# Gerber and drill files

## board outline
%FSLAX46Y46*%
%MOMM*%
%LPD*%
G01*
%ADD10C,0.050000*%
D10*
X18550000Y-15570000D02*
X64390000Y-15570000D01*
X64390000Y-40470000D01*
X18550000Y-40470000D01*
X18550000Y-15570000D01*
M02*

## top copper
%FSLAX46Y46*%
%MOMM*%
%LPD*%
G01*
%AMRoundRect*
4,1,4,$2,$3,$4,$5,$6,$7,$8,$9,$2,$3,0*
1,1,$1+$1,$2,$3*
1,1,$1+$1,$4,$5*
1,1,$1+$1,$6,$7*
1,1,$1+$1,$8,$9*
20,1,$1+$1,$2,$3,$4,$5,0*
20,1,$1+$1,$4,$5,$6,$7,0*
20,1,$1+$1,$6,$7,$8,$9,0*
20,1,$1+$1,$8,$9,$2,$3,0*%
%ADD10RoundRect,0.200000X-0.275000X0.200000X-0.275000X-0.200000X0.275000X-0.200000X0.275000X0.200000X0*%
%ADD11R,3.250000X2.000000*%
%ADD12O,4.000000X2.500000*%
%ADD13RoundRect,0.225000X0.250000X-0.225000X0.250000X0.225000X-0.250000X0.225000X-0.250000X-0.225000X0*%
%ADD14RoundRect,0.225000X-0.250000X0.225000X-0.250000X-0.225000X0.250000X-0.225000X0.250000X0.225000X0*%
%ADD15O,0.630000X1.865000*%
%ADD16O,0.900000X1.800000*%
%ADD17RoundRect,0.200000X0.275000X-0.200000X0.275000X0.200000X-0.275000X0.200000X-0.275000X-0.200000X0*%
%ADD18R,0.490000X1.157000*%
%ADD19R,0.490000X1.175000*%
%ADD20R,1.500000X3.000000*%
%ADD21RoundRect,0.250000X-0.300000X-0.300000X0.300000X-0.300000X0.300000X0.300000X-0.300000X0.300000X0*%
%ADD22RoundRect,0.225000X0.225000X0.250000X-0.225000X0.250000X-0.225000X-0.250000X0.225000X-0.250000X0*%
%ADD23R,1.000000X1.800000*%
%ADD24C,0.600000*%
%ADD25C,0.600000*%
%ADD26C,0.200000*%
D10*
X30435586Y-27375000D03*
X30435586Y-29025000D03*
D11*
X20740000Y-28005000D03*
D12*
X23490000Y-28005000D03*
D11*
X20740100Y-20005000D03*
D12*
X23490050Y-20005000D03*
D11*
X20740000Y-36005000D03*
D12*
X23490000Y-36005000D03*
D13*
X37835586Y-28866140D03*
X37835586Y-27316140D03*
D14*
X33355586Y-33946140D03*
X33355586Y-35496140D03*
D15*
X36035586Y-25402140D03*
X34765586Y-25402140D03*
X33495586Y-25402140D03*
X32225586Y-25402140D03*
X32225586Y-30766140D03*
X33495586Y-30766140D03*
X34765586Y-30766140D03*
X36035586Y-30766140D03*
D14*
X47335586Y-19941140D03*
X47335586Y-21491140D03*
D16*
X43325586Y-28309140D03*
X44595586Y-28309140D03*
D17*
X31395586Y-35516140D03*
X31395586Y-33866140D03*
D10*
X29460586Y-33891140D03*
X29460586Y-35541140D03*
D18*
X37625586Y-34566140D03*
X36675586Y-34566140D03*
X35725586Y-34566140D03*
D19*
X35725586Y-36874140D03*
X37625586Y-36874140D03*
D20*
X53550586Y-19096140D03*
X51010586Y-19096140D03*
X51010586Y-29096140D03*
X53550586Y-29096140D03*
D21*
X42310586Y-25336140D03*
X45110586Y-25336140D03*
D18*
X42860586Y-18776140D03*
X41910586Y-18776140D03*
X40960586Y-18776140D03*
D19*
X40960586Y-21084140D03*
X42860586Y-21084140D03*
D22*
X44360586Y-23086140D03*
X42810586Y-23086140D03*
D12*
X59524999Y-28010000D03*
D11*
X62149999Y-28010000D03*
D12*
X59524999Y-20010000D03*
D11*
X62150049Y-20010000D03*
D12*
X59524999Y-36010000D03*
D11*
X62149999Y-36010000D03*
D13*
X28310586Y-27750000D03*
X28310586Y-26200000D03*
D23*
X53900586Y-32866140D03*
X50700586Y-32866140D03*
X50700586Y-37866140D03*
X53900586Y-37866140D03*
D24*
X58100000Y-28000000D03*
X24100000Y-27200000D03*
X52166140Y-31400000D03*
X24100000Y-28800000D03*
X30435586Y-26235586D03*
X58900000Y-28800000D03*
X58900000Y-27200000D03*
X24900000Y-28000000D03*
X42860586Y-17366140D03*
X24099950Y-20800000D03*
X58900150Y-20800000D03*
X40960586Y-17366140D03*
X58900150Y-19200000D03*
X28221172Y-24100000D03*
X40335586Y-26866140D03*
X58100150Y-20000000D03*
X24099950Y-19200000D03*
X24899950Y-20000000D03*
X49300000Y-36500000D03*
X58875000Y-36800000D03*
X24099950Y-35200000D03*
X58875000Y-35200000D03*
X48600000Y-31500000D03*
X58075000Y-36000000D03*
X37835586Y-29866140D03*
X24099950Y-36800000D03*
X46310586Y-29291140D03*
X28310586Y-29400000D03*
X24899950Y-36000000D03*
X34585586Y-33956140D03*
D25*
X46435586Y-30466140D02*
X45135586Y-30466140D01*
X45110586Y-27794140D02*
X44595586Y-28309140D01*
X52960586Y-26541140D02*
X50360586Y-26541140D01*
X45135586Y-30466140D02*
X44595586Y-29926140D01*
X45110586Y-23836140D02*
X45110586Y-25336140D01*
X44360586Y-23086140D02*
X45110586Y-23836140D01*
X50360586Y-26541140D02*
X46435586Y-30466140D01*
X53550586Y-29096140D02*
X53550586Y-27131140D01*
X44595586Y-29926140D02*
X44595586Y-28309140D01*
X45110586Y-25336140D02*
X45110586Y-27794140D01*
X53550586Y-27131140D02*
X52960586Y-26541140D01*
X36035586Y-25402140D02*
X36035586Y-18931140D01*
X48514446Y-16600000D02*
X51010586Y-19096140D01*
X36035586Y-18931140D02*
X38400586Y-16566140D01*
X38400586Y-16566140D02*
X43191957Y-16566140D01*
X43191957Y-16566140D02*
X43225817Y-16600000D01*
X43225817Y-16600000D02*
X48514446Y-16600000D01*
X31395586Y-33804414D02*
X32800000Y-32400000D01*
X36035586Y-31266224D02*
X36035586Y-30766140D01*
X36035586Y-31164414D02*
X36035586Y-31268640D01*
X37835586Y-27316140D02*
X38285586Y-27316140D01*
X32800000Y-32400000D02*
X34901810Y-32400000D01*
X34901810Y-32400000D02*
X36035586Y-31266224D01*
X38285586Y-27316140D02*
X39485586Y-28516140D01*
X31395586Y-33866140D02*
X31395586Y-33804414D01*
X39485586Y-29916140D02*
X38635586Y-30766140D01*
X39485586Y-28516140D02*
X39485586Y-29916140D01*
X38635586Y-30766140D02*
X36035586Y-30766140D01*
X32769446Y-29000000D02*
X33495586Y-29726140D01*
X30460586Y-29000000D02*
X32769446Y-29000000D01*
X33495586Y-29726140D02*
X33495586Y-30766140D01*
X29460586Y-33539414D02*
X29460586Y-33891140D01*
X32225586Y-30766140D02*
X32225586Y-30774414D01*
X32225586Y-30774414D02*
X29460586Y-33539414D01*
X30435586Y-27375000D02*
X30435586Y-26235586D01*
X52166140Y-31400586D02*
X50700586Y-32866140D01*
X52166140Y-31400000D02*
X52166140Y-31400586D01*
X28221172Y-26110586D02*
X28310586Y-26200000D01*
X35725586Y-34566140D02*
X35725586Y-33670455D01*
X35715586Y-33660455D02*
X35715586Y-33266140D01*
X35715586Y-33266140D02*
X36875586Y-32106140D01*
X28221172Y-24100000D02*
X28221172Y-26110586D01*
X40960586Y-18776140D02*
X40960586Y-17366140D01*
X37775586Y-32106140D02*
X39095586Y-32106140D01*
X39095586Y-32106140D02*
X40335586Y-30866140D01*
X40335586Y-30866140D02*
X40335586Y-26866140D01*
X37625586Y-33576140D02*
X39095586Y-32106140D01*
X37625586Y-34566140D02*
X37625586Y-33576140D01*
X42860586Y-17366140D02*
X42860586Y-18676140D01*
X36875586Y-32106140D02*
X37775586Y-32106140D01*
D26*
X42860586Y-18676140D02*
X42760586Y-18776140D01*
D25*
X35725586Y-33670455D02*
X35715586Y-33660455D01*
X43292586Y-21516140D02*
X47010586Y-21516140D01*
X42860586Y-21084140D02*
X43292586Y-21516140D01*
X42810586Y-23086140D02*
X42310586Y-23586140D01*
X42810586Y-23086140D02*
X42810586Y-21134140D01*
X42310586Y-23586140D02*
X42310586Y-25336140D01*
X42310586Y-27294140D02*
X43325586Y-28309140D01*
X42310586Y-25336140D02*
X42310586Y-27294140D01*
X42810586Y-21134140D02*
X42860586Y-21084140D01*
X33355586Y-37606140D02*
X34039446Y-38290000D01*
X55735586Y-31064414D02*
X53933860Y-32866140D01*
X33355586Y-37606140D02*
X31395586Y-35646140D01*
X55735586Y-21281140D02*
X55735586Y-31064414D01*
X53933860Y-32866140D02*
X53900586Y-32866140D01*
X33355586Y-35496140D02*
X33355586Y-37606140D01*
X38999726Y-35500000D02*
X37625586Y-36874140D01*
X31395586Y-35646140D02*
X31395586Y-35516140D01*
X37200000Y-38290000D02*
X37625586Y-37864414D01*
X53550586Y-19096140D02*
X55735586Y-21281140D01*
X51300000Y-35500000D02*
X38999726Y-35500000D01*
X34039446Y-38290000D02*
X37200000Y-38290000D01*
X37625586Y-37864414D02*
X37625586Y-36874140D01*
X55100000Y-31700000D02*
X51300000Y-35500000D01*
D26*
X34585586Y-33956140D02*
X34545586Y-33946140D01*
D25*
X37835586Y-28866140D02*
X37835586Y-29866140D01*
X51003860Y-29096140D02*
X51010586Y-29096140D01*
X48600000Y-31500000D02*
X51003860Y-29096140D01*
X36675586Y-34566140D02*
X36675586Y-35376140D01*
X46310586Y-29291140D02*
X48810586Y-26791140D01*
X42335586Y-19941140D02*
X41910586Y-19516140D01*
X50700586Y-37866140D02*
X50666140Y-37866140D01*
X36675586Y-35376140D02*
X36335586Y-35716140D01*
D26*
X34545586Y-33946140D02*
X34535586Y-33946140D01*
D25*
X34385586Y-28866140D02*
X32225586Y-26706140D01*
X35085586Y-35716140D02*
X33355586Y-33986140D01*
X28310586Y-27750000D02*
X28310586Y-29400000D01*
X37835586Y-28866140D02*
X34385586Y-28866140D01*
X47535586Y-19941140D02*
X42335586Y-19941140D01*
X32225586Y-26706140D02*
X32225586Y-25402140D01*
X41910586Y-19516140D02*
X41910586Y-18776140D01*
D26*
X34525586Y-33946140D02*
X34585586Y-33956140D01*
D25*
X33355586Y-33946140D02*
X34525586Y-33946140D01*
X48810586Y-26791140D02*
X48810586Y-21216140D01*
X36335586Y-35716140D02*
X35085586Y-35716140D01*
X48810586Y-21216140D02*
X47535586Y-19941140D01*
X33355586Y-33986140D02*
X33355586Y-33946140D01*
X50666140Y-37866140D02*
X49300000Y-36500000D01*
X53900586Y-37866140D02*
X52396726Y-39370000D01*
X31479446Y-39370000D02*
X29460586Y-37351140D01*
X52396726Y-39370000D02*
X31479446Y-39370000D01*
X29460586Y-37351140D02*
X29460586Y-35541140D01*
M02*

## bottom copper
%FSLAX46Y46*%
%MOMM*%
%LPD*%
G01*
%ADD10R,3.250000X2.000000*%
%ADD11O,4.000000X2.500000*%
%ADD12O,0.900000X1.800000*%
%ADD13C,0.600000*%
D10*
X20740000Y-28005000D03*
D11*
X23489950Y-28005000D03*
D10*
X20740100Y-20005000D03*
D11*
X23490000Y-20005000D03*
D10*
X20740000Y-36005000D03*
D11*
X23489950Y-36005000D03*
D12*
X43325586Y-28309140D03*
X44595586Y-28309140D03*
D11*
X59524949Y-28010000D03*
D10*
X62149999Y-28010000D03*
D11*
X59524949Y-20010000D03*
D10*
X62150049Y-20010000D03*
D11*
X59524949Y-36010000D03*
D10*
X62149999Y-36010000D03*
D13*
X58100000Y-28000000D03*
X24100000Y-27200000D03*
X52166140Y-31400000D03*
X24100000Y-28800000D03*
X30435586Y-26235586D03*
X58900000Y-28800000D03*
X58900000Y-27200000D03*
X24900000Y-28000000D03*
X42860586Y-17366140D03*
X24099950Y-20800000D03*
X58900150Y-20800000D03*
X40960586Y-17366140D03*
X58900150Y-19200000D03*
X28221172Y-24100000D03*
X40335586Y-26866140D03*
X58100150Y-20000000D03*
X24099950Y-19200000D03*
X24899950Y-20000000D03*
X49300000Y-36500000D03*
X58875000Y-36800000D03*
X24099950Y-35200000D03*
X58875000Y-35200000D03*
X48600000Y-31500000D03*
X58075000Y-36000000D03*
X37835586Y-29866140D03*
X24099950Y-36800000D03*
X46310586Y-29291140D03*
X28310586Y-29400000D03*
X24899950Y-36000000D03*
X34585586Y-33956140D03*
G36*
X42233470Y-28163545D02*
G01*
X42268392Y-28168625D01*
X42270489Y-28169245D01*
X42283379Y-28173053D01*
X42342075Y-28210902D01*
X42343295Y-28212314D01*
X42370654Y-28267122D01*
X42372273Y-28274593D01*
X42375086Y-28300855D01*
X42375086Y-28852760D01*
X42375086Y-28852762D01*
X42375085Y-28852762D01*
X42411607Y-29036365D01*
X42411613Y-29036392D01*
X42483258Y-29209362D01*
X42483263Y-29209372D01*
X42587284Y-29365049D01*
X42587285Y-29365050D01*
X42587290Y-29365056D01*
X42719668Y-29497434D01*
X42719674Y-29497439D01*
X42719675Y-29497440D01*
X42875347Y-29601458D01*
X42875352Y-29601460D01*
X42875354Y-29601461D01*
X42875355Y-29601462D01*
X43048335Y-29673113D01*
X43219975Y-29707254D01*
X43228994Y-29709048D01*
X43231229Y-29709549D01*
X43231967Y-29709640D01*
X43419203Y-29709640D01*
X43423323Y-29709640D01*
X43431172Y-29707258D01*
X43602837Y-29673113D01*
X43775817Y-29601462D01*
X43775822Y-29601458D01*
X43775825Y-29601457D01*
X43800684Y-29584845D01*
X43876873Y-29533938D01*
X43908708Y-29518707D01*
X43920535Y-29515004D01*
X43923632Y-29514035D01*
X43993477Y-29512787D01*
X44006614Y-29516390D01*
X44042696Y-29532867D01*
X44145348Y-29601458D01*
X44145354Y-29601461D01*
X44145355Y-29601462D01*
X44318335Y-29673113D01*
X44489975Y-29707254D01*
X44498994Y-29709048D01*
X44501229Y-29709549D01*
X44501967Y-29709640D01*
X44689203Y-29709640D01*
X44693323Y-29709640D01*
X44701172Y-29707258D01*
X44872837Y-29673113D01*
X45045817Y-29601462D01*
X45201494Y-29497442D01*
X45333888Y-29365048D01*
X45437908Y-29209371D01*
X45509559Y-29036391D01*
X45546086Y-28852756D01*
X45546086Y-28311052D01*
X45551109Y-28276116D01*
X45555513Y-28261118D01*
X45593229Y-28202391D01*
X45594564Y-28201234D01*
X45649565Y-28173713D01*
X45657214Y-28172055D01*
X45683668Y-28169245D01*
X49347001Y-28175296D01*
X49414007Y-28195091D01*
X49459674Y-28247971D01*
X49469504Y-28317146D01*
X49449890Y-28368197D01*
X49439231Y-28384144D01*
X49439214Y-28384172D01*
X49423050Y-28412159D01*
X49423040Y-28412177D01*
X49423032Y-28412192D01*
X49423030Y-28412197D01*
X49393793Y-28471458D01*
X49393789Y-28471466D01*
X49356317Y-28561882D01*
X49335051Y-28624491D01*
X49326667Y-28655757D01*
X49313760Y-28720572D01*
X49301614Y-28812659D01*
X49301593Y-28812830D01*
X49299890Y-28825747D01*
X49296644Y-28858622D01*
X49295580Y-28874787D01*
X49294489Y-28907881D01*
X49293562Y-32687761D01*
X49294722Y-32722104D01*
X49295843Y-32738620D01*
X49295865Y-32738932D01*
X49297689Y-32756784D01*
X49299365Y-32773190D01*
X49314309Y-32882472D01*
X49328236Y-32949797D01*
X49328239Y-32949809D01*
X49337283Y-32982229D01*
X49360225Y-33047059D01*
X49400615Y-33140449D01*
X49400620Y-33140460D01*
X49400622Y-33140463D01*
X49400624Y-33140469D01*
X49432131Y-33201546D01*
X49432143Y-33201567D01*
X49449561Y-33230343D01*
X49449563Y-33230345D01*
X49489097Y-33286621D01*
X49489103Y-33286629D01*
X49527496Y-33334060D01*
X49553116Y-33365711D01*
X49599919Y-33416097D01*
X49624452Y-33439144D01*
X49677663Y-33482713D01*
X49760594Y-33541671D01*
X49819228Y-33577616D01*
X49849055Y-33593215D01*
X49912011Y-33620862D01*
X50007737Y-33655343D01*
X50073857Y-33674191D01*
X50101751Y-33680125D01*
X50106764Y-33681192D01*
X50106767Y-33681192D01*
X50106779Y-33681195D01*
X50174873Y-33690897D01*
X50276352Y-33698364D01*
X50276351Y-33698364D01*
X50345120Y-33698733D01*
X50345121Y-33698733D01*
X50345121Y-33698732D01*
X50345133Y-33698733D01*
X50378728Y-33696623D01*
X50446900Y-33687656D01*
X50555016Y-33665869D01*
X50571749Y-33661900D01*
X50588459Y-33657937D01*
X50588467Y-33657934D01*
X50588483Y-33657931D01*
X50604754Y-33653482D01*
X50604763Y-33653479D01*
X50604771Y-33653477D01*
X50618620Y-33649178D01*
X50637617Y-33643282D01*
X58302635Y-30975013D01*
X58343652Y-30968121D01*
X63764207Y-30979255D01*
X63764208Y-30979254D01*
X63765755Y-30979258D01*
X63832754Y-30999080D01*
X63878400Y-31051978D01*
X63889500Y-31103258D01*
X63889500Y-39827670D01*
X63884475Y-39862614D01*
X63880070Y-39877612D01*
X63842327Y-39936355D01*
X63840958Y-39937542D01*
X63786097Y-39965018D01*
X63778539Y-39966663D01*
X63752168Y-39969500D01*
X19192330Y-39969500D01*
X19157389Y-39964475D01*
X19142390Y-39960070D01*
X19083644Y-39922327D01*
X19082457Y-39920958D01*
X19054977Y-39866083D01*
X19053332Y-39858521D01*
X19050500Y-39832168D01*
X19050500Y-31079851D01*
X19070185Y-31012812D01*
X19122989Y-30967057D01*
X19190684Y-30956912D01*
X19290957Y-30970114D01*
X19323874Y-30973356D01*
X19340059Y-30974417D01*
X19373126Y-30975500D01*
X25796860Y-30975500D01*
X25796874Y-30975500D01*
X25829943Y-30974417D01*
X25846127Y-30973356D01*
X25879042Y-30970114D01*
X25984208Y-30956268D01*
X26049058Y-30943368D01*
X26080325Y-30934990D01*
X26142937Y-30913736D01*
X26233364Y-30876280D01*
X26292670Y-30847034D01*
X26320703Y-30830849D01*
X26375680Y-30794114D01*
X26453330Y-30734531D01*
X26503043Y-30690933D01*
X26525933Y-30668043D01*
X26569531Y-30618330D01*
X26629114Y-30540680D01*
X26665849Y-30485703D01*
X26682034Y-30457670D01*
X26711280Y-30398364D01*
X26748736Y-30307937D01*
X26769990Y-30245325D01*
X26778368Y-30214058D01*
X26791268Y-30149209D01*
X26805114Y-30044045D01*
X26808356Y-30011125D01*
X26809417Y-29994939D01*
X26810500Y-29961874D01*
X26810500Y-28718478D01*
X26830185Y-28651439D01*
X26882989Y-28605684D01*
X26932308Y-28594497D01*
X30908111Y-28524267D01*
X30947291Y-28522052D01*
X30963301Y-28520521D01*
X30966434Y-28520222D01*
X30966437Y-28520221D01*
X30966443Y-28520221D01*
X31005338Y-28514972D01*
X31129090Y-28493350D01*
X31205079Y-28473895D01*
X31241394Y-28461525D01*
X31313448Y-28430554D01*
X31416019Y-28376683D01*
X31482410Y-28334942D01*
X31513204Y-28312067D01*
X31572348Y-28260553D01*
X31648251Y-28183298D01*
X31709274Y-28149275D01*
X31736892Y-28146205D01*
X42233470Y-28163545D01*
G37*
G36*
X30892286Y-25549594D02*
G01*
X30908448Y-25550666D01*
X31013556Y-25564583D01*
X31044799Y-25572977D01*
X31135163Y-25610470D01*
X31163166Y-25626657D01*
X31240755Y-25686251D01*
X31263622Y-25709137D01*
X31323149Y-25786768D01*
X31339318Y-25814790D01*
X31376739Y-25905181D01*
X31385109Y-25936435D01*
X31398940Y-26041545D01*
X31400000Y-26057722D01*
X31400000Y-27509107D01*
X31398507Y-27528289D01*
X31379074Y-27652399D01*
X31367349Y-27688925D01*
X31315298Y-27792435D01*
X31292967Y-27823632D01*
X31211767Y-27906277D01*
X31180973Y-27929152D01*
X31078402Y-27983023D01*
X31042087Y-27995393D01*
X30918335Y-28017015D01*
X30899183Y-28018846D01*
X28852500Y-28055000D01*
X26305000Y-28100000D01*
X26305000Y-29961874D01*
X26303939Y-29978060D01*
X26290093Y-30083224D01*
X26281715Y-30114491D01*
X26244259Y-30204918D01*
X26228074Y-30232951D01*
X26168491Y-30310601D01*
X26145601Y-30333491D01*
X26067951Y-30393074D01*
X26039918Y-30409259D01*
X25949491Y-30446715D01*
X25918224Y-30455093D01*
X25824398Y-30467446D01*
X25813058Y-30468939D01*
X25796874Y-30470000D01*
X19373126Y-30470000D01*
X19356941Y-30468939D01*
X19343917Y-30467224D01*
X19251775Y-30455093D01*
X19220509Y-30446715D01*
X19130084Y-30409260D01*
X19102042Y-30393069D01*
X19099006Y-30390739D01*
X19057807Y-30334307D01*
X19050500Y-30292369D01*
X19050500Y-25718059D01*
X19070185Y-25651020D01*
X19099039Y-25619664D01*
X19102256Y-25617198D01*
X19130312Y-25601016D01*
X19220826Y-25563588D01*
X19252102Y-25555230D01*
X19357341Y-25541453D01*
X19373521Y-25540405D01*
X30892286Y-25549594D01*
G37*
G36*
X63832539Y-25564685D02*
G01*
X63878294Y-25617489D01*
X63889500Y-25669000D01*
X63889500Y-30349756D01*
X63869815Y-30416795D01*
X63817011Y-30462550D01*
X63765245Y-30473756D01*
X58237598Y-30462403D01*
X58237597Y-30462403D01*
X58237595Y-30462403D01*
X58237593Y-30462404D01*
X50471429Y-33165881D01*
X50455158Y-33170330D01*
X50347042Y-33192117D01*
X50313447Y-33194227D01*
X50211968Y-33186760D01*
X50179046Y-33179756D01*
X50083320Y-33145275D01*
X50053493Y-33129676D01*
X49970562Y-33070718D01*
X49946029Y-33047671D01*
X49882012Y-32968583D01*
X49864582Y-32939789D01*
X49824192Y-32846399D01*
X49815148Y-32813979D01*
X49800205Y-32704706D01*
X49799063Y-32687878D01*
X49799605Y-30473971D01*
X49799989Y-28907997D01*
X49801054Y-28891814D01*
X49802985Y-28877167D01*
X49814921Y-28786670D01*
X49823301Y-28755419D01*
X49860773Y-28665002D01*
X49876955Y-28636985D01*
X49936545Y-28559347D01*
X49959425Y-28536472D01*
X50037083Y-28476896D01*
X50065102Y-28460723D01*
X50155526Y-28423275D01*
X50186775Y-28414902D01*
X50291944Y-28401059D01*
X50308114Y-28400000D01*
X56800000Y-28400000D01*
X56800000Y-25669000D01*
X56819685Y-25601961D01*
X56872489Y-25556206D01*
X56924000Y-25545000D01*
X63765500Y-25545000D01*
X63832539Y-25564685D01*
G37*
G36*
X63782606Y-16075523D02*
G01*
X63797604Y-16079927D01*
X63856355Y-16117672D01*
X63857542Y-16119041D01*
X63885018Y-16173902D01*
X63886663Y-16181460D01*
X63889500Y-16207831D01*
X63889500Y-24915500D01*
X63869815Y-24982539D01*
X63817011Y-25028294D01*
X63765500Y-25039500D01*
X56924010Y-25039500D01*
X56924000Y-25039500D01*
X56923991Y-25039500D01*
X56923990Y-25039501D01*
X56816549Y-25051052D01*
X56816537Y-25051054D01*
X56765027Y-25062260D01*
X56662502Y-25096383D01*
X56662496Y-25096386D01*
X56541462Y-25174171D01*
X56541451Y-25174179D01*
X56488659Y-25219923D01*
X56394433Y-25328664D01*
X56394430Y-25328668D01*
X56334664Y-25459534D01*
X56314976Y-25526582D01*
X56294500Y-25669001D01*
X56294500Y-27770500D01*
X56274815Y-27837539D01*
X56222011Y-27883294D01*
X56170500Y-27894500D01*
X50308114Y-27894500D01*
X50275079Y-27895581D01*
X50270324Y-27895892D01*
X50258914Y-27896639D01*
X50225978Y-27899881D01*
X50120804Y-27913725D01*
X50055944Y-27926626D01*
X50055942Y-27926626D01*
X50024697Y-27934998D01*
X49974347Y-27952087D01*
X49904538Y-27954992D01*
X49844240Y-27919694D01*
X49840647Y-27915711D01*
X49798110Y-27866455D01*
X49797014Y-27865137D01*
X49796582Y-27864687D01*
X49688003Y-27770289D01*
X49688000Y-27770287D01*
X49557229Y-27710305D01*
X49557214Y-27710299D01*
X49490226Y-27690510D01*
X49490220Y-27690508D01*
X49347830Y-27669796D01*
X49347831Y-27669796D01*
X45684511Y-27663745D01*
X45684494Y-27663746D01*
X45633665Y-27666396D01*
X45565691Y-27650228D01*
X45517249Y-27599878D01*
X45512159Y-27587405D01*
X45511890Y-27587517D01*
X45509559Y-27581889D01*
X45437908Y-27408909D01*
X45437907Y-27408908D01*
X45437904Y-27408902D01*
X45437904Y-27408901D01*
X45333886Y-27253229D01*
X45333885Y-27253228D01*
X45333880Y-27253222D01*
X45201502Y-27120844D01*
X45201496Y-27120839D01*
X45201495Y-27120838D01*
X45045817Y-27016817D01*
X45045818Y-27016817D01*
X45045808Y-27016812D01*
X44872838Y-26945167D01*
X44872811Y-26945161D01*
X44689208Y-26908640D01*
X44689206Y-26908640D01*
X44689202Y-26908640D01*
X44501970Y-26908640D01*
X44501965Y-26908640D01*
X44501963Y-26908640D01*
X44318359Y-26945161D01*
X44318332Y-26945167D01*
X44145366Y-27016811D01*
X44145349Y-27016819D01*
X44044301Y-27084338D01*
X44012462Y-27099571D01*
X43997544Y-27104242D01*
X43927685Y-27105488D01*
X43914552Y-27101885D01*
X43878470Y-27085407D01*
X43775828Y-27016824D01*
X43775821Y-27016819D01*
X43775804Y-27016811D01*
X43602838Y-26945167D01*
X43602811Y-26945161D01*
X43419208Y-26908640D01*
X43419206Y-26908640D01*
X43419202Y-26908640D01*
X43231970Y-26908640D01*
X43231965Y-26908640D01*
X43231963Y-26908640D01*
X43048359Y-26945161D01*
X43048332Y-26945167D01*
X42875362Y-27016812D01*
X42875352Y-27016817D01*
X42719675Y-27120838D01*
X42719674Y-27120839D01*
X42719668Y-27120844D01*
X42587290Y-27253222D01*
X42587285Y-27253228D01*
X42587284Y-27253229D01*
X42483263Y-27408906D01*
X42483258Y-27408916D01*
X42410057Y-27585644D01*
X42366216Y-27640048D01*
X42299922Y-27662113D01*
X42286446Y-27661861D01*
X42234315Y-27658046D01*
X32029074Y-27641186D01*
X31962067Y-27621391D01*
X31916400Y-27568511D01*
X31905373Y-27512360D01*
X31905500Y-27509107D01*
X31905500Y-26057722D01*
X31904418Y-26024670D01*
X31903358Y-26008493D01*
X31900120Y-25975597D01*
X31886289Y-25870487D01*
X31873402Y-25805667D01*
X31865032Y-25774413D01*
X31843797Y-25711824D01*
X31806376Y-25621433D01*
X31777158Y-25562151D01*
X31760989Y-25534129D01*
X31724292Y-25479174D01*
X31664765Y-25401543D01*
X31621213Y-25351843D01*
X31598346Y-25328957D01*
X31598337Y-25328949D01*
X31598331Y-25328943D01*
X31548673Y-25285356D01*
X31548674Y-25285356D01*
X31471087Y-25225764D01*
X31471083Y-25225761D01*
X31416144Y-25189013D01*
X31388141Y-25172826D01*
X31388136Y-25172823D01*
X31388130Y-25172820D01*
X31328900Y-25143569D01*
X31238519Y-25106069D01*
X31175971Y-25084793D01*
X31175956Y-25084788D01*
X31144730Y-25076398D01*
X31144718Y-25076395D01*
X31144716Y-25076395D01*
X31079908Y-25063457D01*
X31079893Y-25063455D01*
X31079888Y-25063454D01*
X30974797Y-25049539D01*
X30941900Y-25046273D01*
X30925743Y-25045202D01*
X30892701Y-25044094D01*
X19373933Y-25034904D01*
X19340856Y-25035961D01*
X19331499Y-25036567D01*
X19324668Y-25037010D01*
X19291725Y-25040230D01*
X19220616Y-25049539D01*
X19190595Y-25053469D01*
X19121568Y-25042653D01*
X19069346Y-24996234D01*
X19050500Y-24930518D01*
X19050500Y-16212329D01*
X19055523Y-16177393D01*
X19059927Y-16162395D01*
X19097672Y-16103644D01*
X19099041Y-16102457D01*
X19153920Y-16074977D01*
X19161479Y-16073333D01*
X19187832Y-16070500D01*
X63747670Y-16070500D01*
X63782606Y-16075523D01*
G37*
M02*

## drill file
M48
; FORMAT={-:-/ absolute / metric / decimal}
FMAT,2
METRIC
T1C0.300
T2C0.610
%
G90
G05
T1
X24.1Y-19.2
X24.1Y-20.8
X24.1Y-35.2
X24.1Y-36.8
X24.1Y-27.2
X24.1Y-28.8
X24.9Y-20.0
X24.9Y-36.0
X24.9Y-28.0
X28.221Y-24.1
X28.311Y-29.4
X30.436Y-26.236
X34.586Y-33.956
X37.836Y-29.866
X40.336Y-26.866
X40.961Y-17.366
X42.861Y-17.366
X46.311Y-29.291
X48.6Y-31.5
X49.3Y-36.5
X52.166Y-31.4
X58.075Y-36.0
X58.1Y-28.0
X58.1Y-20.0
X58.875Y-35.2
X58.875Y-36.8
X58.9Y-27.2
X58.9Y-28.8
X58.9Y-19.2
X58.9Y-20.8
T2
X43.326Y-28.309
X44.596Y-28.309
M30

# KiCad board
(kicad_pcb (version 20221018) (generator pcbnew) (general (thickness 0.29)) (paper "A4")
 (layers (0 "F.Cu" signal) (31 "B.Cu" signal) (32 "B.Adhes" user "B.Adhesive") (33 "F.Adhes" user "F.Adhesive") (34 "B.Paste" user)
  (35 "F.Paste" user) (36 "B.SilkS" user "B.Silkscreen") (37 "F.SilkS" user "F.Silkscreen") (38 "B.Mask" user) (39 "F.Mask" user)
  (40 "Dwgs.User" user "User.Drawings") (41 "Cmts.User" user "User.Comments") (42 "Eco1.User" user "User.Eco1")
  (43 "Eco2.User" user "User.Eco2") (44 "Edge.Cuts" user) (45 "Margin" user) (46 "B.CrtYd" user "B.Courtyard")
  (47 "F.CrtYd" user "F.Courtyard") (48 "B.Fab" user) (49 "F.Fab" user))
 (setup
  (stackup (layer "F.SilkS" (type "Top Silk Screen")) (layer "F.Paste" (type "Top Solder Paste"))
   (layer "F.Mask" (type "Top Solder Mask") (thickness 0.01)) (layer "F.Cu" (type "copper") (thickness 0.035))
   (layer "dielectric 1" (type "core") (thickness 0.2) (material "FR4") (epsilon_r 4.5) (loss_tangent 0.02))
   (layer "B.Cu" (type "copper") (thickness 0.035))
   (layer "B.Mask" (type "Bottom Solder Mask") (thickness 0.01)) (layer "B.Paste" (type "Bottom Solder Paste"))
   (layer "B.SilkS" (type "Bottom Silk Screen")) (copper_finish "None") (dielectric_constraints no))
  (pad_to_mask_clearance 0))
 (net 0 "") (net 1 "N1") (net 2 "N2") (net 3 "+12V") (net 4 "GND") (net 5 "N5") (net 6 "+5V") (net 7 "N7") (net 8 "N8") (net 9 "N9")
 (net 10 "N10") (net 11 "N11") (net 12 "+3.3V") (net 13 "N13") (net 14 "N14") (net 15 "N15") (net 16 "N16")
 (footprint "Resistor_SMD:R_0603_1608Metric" (layer "F.Cu") (at 30.435586 28.2 -90)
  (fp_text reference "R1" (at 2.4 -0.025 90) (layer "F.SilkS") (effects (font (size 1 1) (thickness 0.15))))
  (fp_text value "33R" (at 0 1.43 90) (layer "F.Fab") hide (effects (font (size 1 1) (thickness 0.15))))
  (pad "1" smd roundrect (at -0.825 0 270) (size 0.8 0.95) (layers "F.Cu" "F.Paste" "F.Mask") (roundrect_rratio 0.25) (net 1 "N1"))
  (pad "2" smd roundrect (at 0.825 0 270) (size 0.8 0.95) (layers "F.Cu" "F.Paste" "F.Mask") (roundrect_rratio 0.25) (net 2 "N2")))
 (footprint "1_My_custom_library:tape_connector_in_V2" (layer "F.Cu") (at 23.49 28.005)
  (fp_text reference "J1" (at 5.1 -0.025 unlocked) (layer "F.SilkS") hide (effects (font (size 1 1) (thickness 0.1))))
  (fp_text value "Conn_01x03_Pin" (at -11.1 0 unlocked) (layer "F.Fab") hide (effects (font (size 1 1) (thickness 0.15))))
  (pad "1" smd rect (at -2.75 0) (size 3.25 2) (layers "F.Cu" "F.Mask") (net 1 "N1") (thermal_bridge_angle 45))
  (pad "1" smd rect (at -2.75 0) (size 3.25 2) (layers "B.Cu" "B.Paste" "B.Mask") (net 1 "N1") (thermal_bridge_angle 45))
  (pad "1" smd oval (at -0.00005 0) (size 4 2.5) (layers "B.Cu" "B.Paste" "B.Mask") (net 1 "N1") (thermal_bridge_angle 45))
  (pad "1" smd oval (at 0 0) (size 4 2.5) (layers "F.Cu" "F.Mask") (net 1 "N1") (thermal_bridge_angle 45))
  (pad "2" smd rect (at -2.7499 -8) (size 3.25 2) (layers "F.Cu" "F.Mask") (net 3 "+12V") (thermal_bridge_angle 45))
  (pad "2" smd rect (at -2.7499 -8) (size 3.25 2) (layers "B.Cu" "B.Paste" "B.Mask") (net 3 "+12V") (thermal_bridge_angle 45))
  (pad "2" smd oval (at 0 -8) (size 4 2.5) (layers "B.Cu" "B.Paste" "B.Mask") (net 3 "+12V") (thermal_bridge_angle 45))
  (pad "2" smd oval (at 0.00005 -8) (size 4 2.5) (layers "F.Cu" "F.Mask") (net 3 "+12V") (thermal_bridge_angle 45))
  (pad "3" smd rect (at -2.75 8) (size 3.25 2) (layers "F.Cu" "F.Mask") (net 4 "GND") (thermal_bridge_angle 45))
  (pad "3" smd rect (at -2.75 8) (size 3.25 2) (layers "B.Cu" "B.Paste" "B.Mask") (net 4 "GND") (thermal_bridge_angle 45))
  (pad "3" smd oval (at -0.00005 8) (size 4 2.5) (layers "B.Cu" "B.Paste" "B.Mask") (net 4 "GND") (thermal_bridge_angle 45))
  (pad "3" smd oval (at 0 8) (size 4 2.5) (layers "F.Cu" "F.Mask") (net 4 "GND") (thermal_bridge_angle 45)))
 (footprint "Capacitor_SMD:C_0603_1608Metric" (layer "F.Cu") (at 37.835586 28.09114 90)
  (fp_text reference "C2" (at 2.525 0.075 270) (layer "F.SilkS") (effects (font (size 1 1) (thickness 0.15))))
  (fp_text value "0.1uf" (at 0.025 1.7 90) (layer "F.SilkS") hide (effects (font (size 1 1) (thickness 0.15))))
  (pad "1" smd roundrect (at -0.775 0 90) (size 0.9 0.95) (layers "F.Cu" "F.Paste" "F.Mask") (roundrect_rratio 0.25) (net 4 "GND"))
  (pad "2" smd roundrect (at 0.775 0 90) (size 0.9 0.95) (layers "F.Cu" "F.Paste" "F.Mask") (roundrect_rratio 0.25) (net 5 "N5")))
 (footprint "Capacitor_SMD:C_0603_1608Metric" (layer "F.Cu") (at 33.355586 34.72114 -90)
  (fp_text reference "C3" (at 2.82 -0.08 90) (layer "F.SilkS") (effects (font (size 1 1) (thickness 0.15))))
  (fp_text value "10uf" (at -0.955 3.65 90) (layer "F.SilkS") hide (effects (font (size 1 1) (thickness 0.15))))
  (pad "1" smd roundrect (at -0.775 0 270) (size 0.9 0.95) (layers "F.Cu" "F.Paste" "F.Mask") (roundrect_rratio 0.25) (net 4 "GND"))
  (pad "2" smd roundrect (at 0.775 0 270) (size 0.9 0.95) (layers "F.Cu" "F.Paste" "F.Mask") (roundrect_rratio 0.25) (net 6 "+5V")))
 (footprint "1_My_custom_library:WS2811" (layer "F.Cu") (at 34.130586 28.08414 180)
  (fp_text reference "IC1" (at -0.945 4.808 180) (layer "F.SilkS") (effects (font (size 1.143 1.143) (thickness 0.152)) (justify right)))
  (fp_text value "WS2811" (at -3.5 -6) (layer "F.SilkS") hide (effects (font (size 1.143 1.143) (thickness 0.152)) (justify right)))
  (pad "1" smd oval (at -1.905 2.682 180) (size 0.63 1.865) (layers "F.Cu" "F.Paste" "F.Mask") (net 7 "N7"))
  (pad "2" smd oval (at -0.635 2.682 180) (size 0.63 1.865) (layers "F.Cu" "F.Paste" "F.Mask") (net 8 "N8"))
  (pad "3" smd oval (at 0.635 2.682 180) (size 0.63 1.865) (layers "F.Cu" "F.Paste" "F.Mask") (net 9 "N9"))
  (pad "4" smd oval (at 1.905 2.682 180) (size 0.63 1.865) (layers "F.Cu" "F.Paste" "F.Mask") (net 4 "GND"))
  (pad "5" smd oval (at 1.905 -2.682 180) (size 0.63 1.865) (layers "F.Cu" "F.Paste" "F.Mask") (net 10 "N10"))
  (pad "6" smd oval (at 0.635 -2.682 180) (size 0.63 1.865) (layers "F.Cu" "F.Paste" "F.Mask") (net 2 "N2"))
  (pad "7" smd oval (at -0.635 -2.682 180) (size 0.63 1.865) (layers "F.Cu" "F.Paste" "F.Mask") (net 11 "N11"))
  (pad "8" smd oval (at -1.905 -2.682 180) (size 0.63 1.865) (layers "F.Cu" "F.Paste" "F.Mask") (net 5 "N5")))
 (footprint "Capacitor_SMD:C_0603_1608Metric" (layer "F.Cu") (at 47.335586 20.71614 -90)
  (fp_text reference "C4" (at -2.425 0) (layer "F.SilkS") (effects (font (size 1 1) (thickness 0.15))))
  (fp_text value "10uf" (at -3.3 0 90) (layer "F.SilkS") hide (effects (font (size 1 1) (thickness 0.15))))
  (pad "1" smd roundrect (at -0.775 0 270) (size 0.9 0.95) (layers "F.Cu" "F.Paste" "F.Mask") (roundrect_rratio 0.25) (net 4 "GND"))
  (pad "2" smd roundrect (at 0.775 0 270) (size 0.9 0.95) (layers "F.Cu" "F.Paste" "F.Mask") (roundrect_rratio 0.25) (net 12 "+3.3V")))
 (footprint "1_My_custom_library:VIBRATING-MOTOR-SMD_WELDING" (layer "F.Cu") (at 43.960586 28.30914 180)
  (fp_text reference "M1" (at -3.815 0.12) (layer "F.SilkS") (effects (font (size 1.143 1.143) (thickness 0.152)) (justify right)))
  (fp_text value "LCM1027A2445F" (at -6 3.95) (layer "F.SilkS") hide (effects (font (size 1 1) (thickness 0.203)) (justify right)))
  (pad "1" thru_hole oval (at 0.635 0 180) (size 0.9 1.8) (drill 0.61) (layers "*.Cu" "*.Paste" "*.Mask") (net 12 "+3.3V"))
  (pad "2" thru_hole oval (at -0.635 0 180) (size 0.9 1.8) (drill 0.61) (layers "*.Cu" "*.Paste" "*.Mask") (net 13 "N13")))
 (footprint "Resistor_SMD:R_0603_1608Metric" (layer "F.Cu") (at 31.395586 34.69114 90)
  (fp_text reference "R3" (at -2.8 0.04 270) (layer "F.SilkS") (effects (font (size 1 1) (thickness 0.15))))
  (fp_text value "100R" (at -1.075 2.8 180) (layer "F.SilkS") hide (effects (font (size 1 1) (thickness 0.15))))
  (pad "1" smd roundrect (at -0.825 0 90) (size 0.8 0.95) (layers "F.Cu" "F.Paste" "F.Mask") (roundrect_rratio 0.25) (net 6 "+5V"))
  (pad "2" smd roundrect (at 0.825 0 90) (size 0.8 0.95) (layers "F.Cu" "F.Paste" "F.Mask") (roundrect_rratio 0.25) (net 5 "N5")))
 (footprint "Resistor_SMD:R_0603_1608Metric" (layer "F.Cu") (at 29.460586 34.71614 -90)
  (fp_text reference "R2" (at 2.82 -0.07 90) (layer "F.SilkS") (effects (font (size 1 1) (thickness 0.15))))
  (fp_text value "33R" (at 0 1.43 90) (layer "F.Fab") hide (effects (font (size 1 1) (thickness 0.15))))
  (pad "1" smd roundrect (at -0.825 0 270) (size 0.8 0.95) (layers "F.Cu" "F.Paste" "F.Mask") (roundrect_rratio 0.25) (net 10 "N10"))
  (pad "2" smd roundrect (at 0.825 0 270) (size 0.8 0.95) (layers "F.Cu" "F.Paste" "F.Mask") (roundrect_rratio 0.25) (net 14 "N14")))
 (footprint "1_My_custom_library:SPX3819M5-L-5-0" (layer "F.Cu") (at 36.675586 35.72014 180)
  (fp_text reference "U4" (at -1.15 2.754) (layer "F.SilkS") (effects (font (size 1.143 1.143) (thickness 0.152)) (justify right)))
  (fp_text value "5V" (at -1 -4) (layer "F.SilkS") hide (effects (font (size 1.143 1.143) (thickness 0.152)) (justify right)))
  (pad "1" smd rect (at -0.95 1.154 180) (size 0.49 1.157) (layers "F.Cu" "F.Paste" "F.Mask") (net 3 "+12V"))
  (pad "2" smd rect (at 0 1.154 180) (size 0.49 1.157) (layers "F.Cu" "F.Paste" "F.Mask") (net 4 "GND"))
  (pad "3" smd rect (at 0.95 1.154 180) (size 0.49 1.157) (layers "F.Cu" "F.Paste" "F.Mask") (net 3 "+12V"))
  (pad "4" smd rect (at 0.95 -1.154 180) (size 0.49 1.175) (layers "F.Cu" "F.Paste" "F.Mask") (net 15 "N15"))
  (pad "5" smd rect (at -0.95 -1.154 180) (size 0.49 1.175) (layers "F.Cu" "F.Paste" "F.Mask") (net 6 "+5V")))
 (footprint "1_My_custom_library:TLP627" (layer "F.Cu") (at 52.280586 24.09614 180)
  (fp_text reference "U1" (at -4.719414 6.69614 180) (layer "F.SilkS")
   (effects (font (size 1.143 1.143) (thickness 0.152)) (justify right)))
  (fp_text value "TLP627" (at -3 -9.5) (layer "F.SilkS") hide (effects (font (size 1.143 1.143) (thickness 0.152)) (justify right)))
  (pad "1" smd rect (at -1.27 5) (size 1.5 3) (layers "F.Cu" "F.Paste" "F.Mask") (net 6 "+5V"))
  (pad "2" smd rect (at 1.27 5) (size 1.5 3) (layers "F.Cu" "F.Paste" "F.Mask") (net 7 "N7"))
  (pad "3" smd rect (at 1.27 -5) (size 1.5 3) (layers "F.Cu" "F.Paste" "F.Mask") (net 4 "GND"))
  (pad "4" smd rect (at -1.27 -5) (size 1.5 3) (layers "F.Cu" "F.Paste" "F.Mask") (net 13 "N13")))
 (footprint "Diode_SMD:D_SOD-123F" (layer "F.Cu") (at 43.710586 25.33614)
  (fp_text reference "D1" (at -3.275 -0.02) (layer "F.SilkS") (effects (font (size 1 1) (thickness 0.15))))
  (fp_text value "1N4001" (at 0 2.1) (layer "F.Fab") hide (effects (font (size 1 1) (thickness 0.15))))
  (pad "1" smd roundrect (at -1.4 0) (size 1.1 1.1) (layers "F.Cu" "F.Paste" "F.Mask") (roundrect_rratio 0.2272727273) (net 12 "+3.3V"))
  (pad "2" smd roundrect (at 1.4 0) (size 1.1 1.1) (layers "F.Cu" "F.Paste" "F.Mask") (roundrect_rratio 0.2272727273) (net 13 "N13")))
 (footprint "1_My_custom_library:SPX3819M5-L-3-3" (layer "F.Cu") (at 41.910586 19.93014 180)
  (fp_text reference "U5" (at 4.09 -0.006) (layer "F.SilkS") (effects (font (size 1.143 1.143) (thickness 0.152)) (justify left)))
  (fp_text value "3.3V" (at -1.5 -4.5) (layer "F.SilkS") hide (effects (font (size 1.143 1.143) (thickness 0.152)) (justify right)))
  (pad "1" smd rect (at -0.95 1.154 180) (size 0.49 1.157) (layers "F.Cu" "F.Paste" "F.Mask") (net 3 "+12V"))
  (pad "2" smd rect (at 0 1.154 180) (size 0.49 1.157) (layers "F.Cu" "F.Paste" "F.Mask") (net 4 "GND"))
  (pad "3" smd rect (at 0.95 1.154 180) (size 0.49 1.157) (layers "F.Cu" "F.Paste" "F.Mask") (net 3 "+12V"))
  (pad "4" smd rect (at 0.95 -1.154 180) (size 0.49 1.175) (layers "F.Cu" "F.Paste" "F.Mask") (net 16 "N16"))
  (pad "5" smd rect (at -0.95 -1.154 180) (size 0.49 1.175) (layers "F.Cu" "F.Paste" "F.Mask") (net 12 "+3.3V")))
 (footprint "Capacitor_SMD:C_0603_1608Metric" (layer "F.Cu") (at 43.585586 23.08614 180)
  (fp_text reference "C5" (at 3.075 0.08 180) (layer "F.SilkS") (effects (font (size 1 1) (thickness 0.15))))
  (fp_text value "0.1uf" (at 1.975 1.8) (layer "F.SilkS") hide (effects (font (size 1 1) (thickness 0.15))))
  (pad "1" smd roundrect (at -0.775 0 180) (size 0.9 0.95) (layers "F.Cu" "F.Paste" "F.Mask") (roundrect_rratio 0.25) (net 13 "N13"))
  (pad "2" smd roundrect (at 0.775 0 180) (size 0.9 0.95) (layers "F.Cu" "F.Paste" "F.Mask") (roundrect_rratio 0.25) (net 12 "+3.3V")))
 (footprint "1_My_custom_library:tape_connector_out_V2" (layer "F.Cu") (at 59.509999 28.01)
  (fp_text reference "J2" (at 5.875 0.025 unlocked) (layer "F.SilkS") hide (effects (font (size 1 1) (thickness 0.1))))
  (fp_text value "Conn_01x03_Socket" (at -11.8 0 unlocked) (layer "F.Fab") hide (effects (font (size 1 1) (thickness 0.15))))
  (pad "1" smd oval (at 0.01495 0) (size 4 2.5) (layers "B.Cu" "B.Paste" "B.Mask") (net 1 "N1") (thermal_bridge_angle 45))
  (pad "1" smd oval (at 0.015 0) (size 4 2.5) (layers "F.Cu" "F.Paste" "F.Mask") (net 1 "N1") (solder_paste_margin -4.0132)
   (thermal_bridge_angle 45))
  (pad "1" smd rect (at 2.64 0) (size 3.25 2) (layers "F.Cu" "F.Mask") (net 1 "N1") (thermal_bridge_angle 45))
  (pad "1" smd rect (at 2.64 0) (size 3.25 2) (layers "B.Cu" "B.Paste" "B.Mask") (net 1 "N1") (thermal_bridge_angle 45))
  (pad "2" smd oval (at 0.01495 -8) (size 4 2.5) (layers "B.Cu" "B.Paste" "B.Mask") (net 3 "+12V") (thermal_bridge_angle 45))
  (pad "2" smd oval (at 0.015 -8) (size 4 2.5) (layers "F.Cu" "F.Paste" "F.Mask") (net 3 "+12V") (solder_paste_margin -4.0132)
   (thermal_bridge_angle 45))
  (pad "2" smd rect (at 2.64005 -8) (size 3.25 2) (layers "F.Cu" "F.Mask") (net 3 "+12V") (thermal_bridge_angle 45))
  (pad "2" smd rect (at 2.64005 -8) (size 3.25 2) (layers "B.Cu" "B.Paste" "B.Mask") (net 3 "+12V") (thermal_bridge_angle 45))
  (pad "3" smd oval (at 0.01495 8) (size 4 2.5) (layers "B.Cu" "B.Paste" "B.Mask") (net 4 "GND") (thermal_bridge_angle 45))
  (pad "3" smd oval (at 0.015 8) (size 4 2.5) (layers "F.Cu" "F.Paste" "F.Mask") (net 4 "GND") (solder_paste_margin -4.0132)
   (thermal_bridge_angle 45))
  (pad "3" smd rect (at 2.64 8) (size 3.25 2) (layers "F.Cu" "F.Mask") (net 4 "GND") (thermal_bridge_angle 45))
  (pad "3" smd rect (at 2.64 8) (size 3.25 2) (layers "B.Cu" "B.Paste" "B.Mask") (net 4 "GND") (thermal_bridge_angle 45)))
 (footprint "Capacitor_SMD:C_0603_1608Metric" (layer "F.Cu") (at 28.310586 26.975 90)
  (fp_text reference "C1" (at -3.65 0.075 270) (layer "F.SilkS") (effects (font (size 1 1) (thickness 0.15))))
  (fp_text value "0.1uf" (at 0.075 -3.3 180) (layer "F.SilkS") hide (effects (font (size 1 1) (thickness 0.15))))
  (pad "1" smd roundrect (at -0.775 0 90) (size 0.9 0.95) (layers "F.Cu" "F.Paste" "F.Mask") (roundrect_rratio 0.25) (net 4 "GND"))
  (pad "2" smd roundrect (at 0.775 0 90) (size 0.9 0.95) (layers "F.Cu" "F.Paste" "F.Mask") (roundrect_rratio 0.25) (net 3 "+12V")))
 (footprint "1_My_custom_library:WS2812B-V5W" (layer "F.Cu") (at 52.300586 35.36614 -90)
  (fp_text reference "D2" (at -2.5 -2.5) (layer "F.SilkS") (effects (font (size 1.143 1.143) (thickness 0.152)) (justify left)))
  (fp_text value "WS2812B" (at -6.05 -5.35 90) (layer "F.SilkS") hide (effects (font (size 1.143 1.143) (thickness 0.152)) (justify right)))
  (pad "1" smd rect (at -2.5 -1.6 90) (size 1.8 1) (layers "F.Cu" "F.Paste" "F.Mask") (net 6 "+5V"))
  (pad "2" smd rect (at -2.5 1.6 90) (size 1.8 1) (layers "F.Cu" "F.Paste" "F.Mask") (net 1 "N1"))
  (pad "3" smd rect (at 2.5 1.6 90) (size 1.8 1) (layers "F.Cu" "F.Paste" "F.Mask") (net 4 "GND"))
  (pad "4" smd rect (at 2.5 -1.6 90) (size 1.8 1) (layers "F.Cu" "F.Paste" "F.Mask") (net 14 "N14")))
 (gr_rect (start 18.55 15.57) (end 64.39 40.47) (stroke (width 0.05) (type default)) (fill none) (layer "Edge.Cuts"))
 (segment (start 46.435586 30.46614) (end 45.135586 30.46614) (width 0.6) (layer "F.Cu") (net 13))
 (segment (start 45.110586 27.79414) (end 44.595586 28.30914) (width 0.6) (layer "F.Cu") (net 13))
 (segment (start 52.960586 26.54114) (end 50.360586 26.54114) (width 0.6) (layer "F.Cu") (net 13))
 (segment (start 45.135586 30.46614) (end 44.595586 29.92614) (width 0.6) (layer "F.Cu") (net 13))
 (segment (start 45.110586 23.83614) (end 45.110586 25.33614) (width 0.6) (layer "F.Cu") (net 13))
 (segment (start 44.360586 23.08614) (end 45.110586 23.83614) (width 0.6) (layer "F.Cu") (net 13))
 (segment (start 50.360586 26.54114) (end 46.435586 30.46614) (width 0.6) (layer "F.Cu") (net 13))
 (segment (start 53.550586 29.09614) (end 53.550586 27.13114) (width 0.6) (layer "F.Cu") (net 13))
 (segment (start 44.595586 29.92614) (end 44.595586 28.30914) (width 0.6) (layer "F.Cu") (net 13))
 (segment (start 45.110586 25.33614) (end 45.110586 27.79414) (width 0.6) (layer "F.Cu") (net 13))
 (segment (start 53.550586 27.13114) (end 52.960586 26.54114) (width 0.6) (layer "F.Cu") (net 13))
 (segment (start 36.035586 25.40214) (end 36.035586 18.93114) (width 0.6) (layer "F.Cu") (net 7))
 (segment (start 48.514446 16.6) (end 51.010586 19.09614) (width 0.6) (layer "F.Cu") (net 7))
 (segment (start 36.035586 18.93114) (end 38.400586 16.56614) (width 0.6) (layer "F.Cu") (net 7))
 (segment (start 38.400586 16.56614) (end 43.191957 16.56614) (width 0.6) (layer "F.Cu") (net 7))
 (segment (start 43.191957 16.56614) (end 43.225817 16.6) (width 0.6) (layer "F.Cu") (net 7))
 (segment (start 43.225817 16.6) (end 48.514446 16.6) (width 0.6) (layer "F.Cu") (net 7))
 (segment (start 31.395586 33.804414) (end 32.8 32.4) (width 0.6) (layer "F.Cu") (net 5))
 (segment (start 36.035586 31.266224) (end 36.035586 30.76614) (width 0.6) (layer "F.Cu") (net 5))
 (segment (start 36.035586 31.164414) (end 36.035586 31.26864) (width 0.6) (layer "F.Cu") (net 5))
 (segment (start 37.835586 27.31614) (end 38.285586 27.31614) (width 0.6) (layer "F.Cu") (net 5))
 (segment (start 32.8 32.4) (end 34.90181 32.4) (width 0.6) (layer "F.Cu") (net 5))
 (segment (start 34.90181 32.4) (end 36.035586 31.266224) (width 0.6) (layer "F.Cu") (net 5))
 (segment (start 38.285586 27.31614) (end 39.485586 28.51614) (width 0.6) (layer "F.Cu") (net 5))
 (segment (start 31.395586 33.86614) (end 31.395586 33.804414) (width 0.6) (layer "F.Cu") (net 5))
 (segment (start 39.485586 29.91614) (end 38.635586 30.76614) (width 0.6) (layer "F.Cu") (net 5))
 (segment (start 39.485586 28.51614) (end 39.485586 29.91614) (width 0.6) (layer "F.Cu") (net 5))
 (segment (start 38.635586 30.76614) (end 36.035586 30.76614) (width 0.6) (layer "F.Cu") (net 5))
 (segment (start 32.769446 29) (end 33.495586 29.72614) (width 0.6) (layer "F.Cu") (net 2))
 (segment (start 30.460586 29) (end 32.769446 29) (width 0.6) (layer "F.Cu") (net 2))
 (segment (start 33.495586 29.72614) (end 33.495586 30.76614) (width 0.6) (layer "F.Cu") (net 2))
 (segment (start 29.460586 33.539414) (end 29.460586 33.89114) (width 0.6) (layer "F.Cu") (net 10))
 (segment (start 32.225586 30.76614) (end 32.225586 30.774414) (width 0.6) (layer "F.Cu") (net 10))
 (segment (start 32.225586 30.774414) (end 29.460586 33.539414) (width 0.6) (layer "F.Cu") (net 10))
 (segment (start 30.435586 27.375) (end 30.435586 26.235586) (width 0.6) (layer "F.Cu") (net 1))
 (segment (start 52.16614 31.400586) (end 50.700586 32.86614) (width 0.6) (layer "F.Cu") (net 1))
 (segment (start 52.16614 31.4) (end 52.16614 31.400586) (width 0.6) (layer "F.Cu") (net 1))
 (via (at 58.1 28) (size 0.6) (drill 0.3) (layers "F.Cu" "B.Cu") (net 1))
 (via (at 24.1 27.2) (size 0.6) (drill 0.3) (layers "F.Cu" "B.Cu") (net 1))
 (via (at 52.16614 31.4) (size 0.6) (drill 0.3) (layers "F.Cu" "B.Cu") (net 1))
 (via (at 24.1 28.8) (size 0.6) (drill 0.3) (layers "F.Cu" "B.Cu") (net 1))
 (via (at 30.435586 26.235586) (size 0.6) (drill 0.3) (layers "F.Cu" "B.Cu") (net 1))
 (via (at 58.9 28.8) (size 0.6) (drill 0.3) (layers "F.Cu" "B.Cu") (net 1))
 (via (at 58.9 27.2) (size 0.6) (drill 0.3) (layers "F.Cu" "B.Cu") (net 1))
 (via (at 24.9 28) (size 0.6) (drill 0.3) (layers "F.Cu" "B.Cu") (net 1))
 (segment (start 28.221172 26.110586) (end 28.310586 26.2) (width 0.6) (layer "F.Cu") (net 3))
 (segment (start 35.725586 34.56614) (end 35.725586 33.670455) (width 0.6) (layer "F.Cu") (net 3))
 (segment (start 35.715586 33.660455) (end 35.715586 33.26614) (width 0.6) (layer "F.Cu") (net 3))
 (segment (start 35.715586 33.26614) (end 36.875586 32.10614) (width 0.6) (layer "F.Cu") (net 3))
 (segment (start 28.221172 24.1) (end 28.221172 26.110586) (width 0.6) (layer "F.Cu") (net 3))
 (segment (start 40.960586 18.77614) (end 40.960586 17.36614) (width 0.6) (layer "F.Cu") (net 3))
 (segment (start 37.775586 32.10614) (end 39.095586 32.10614) (width 0.6) (layer "F.Cu") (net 3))
 (segment (start 39.095586 32.10614) (end 40.335586 30.86614) (width 0.6) (layer "F.Cu") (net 3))
 (segment (start 40.335586 30.86614) (end 40.335586 26.86614) (width 0.6) (layer "F.Cu") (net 3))
 (segment (start 37.625586 33.57614) (end 39.095586 32.10614) (width 0.6) (layer "F.Cu") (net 3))
 (segment (start 37.625586 34.56614) (end 37.625586 33.57614) (width 0.6) (layer "F.Cu") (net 3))
 (segment (start 42.860586 17.36614) (end 42.860586 18.67614) (width 0.6) (layer "F.Cu") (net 3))
 (segment (start 36.875586 32.10614) (end 37.775586 32.10614) (width 0.6) (layer "F.Cu") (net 3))
 (segment (start 42.860586 18.67614) (end 42.760586 18.77614) (width 0.2) (layer "F.Cu") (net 3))
 (segment (start 35.725586 33.670455) (end 35.715586 33.660455) (width 0.6) (layer "F.Cu") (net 3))
 (via (at 42.860586 17.36614) (size 0.6) (drill 0.3) (layers "F.Cu" "B.Cu") (free) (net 3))
 (via (at 24.09995 20.8) (size 0.6) (drill 0.3) (layers "F.Cu" "B.Cu") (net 3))
 (via (at 58.90015 20.8) (size 0.6) (drill 0.3) (layers "F.Cu" "B.Cu") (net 3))
 (via (at 40.960586 17.36614) (size 0.6) (drill 0.3) (layers "F.Cu" "B.Cu") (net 3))
 (via (at 58.90015 19.2) (size 0.6) (drill 0.3) (layers "F.Cu" "B.Cu") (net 3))
 (via (at 28.221172 24.1) (size 0.6) (drill 0.3) (layers "F.Cu" "B.Cu") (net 3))
 (via (at 40.335586 26.86614) (size 0.6) (drill 0.3) (layers "F.Cu" "B.Cu") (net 3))
 (via (at 58.10015 20) (size 0.6) (drill 0.3) (layers "F.Cu" "B.Cu") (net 3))
 (via (at 24.09995 19.2) (size 0.6) (drill 0.3) (layers "F.Cu" "B.Cu") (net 3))
 (via (at 24.89995 20) (size 0.6) (drill 0.3) (layers "F.Cu" "B.Cu") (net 3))
 (segment (start 43.292586 21.51614) (end 47.010586 21.51614) (width 0.6) (layer "F.Cu") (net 12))
 (segment (start 42.860586 21.08414) (end 43.292586 21.51614) (width 0.6) (layer "F.Cu") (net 12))
 (segment (start 42.810586 23.08614) (end 42.310586 23.58614) (width 0.6) (layer "F.Cu") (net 12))
 (segment (start 42.810586 23.08614) (end 42.810586 21.13414) (width 0.6) (layer "F.Cu") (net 12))
 (segment (start 42.310586 23.58614) (end 42.310586 25.33614) (width 0.6) (layer "F.Cu") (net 12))
 (segment (start 42.310586 27.29414) (end 43.325586 28.30914) (width 0.6) (layer "F.Cu") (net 12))
 (segment (start 42.310586 25.33614) (end 42.310586 27.29414) (width 0.6) (layer "F.Cu") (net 12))
 (segment (start 42.810586 21.13414) (end 42.860586 21.08414) (width 0.6) (layer "F.Cu") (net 12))
 (segment (start 33.355586 37.60614) (end 34.039446 38.29) (width 0.6) (layer "F.Cu") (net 6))
 (segment (start 55.735586 31.064414) (end 53.93386 32.86614) (width 0.6) (layer "F.Cu") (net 6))
 (segment (start 33.355586 37.60614) (end 31.395586 35.64614) (width 0.6) (layer "F.Cu") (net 6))
 (segment (start 55.735586 21.28114) (end 55.735586 31.064414) (width 0.6) (layer "F.Cu") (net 6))
 (segment (start 53.93386 32.86614) (end 53.900586 32.86614) (width 0.6) (layer "F.Cu") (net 6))
 (segment (start 33.355586 35.49614) (end 33.355586 37.60614) (width 0.6) (layer "F.Cu") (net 6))
 (segment (start 38.999726 35.5) (end 37.625586 36.87414) (width 0.6) (layer "F.Cu") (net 6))
 (segment (start 31.395586 35.64614) (end 31.395586 35.51614) (width 0.6) (layer "F.Cu") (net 6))
 (segment (start 37.2 38.29) (end 37.625586 37.864414) (width 0.6) (layer "F.Cu") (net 6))
 (segment (start 53.550586 19.09614) (end 55.735586 21.28114) (width 0.6) (layer "F.Cu") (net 6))
 (segment (start 51.3 35.5) (end 38.999726 35.5) (width 0.6) (layer "F.Cu") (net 6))
 (segment (start 34.039446 38.29) (end 37.2 38.29) (width 0.6) (layer "F.Cu") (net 6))
 (segment (start 37.625586 37.864414) (end 37.625586 36.87414) (width 0.6) (layer "F.Cu") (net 6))
 (segment (start 55.1 31.7) (end 51.3 35.5) (width 0.6) (layer "F.Cu") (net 6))
 (segment (start 34.585586 33.95614) (end 34.545586 33.94614) (width 0.2) (layer "F.Cu") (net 4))
 (segment (start 37.835586 28.86614) (end 37.835586 29.86614) (width 0.6) (layer "F.Cu") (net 4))
 (segment (start 51.00386 29.09614) (end 51.010586 29.09614) (width 0.6) (layer "F.Cu") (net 4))
 (segment (start 48.6 31.5) (end 51.00386 29.09614) (width 0.6) (layer "F.Cu") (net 4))
 (segment (start 36.675586 34.56614) (end 36.675586 35.37614) (width 0.6) (layer "F.Cu") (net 4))
 (segment (start 46.310586 29.29114) (end 48.810586 26.79114) (width 0.6) (layer "F.Cu") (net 4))
 (segment (start 42.335586 19.94114) (end 41.910586 19.51614) (width 0.6) (layer "F.Cu") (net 4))
 (segment (start 50.700586 37.86614) (end 50.66614 37.86614) (width 0.6) (layer "F.Cu") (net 4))
 (segment (start 36.675586 35.37614) (end 36.335586 35.71614) (width 0.6) (layer "F.Cu") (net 4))
 (segment (start 34.545586 33.94614) (end 34.535586 33.94614) (width 0.2) (layer "F.Cu") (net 4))
 (segment (start 34.385586 28.86614) (end 32.225586 26.70614) (width 0.6) (layer "F.Cu") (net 4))
 (segment (start 35.085586 35.71614) (end 33.355586 33.98614) (width 0.6) (layer "F.Cu") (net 4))
 (segment (start 28.310586 27.75) (end 28.310586 29.4) (width 0.6) (layer "F.Cu") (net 4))
 (segment (start 37.835586 28.86614) (end 34.385586 28.86614) (width 0.6) (layer "F.Cu") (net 4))
 (segment (start 47.535586 19.94114) (end 42.335586 19.94114) (width 0.6) (layer "F.Cu") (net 4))
 (segment (start 32.225586 26.70614) (end 32.225586 25.40214) (width 0.6) (layer "F.Cu") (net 4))
 (segment (start 41.910586 19.51614) (end 41.910586 18.77614) (width 0.6) (layer "F.Cu") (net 4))
 (segment (start 34.525586 33.94614) (end 34.585586 33.95614) (width 0.2) (layer "F.Cu") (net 4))
 (segment (start 33.355586 33.94614) (end 34.525586 33.94614) (width 0.6) (layer "F.Cu") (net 4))
 (segment (start 48.810586 26.79114) (end 48.810586 21.21614) (width 0.6) (layer "F.Cu") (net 4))
 (segment (start 36.335586 35.71614) (end 35.085586 35.71614) (width 0.6) (layer "F.Cu") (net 4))
 (segment (start 48.810586 21.21614) (end 47.535586 19.94114) (width 0.6) (layer "F.Cu") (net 4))
 (segment (start 33.355586 33.98614) (end 33.355586 33.94614) (width 0.6) (layer "F.Cu") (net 4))
 (segment (start 50.66614 37.86614) (end 49.3 36.5) (width 0.6) (layer "F.Cu") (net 4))
 (via (at 49.3 36.5) (size 0.6) (drill 0.3) (layers "F.Cu" "B.Cu") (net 4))
 (via (at 58.875 36.8) (size 0.6) (drill 0.3) (layers "F.Cu" "B.Cu") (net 4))
 (via (at 24.09995 35.2) (size 0.6) (drill 0.3) (layers "F.Cu" "B.Cu") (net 4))
 (via (at 58.875 35.2) (size 0.6) (drill 0.3) (layers "F.Cu" "B.Cu") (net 4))
 (via (at 48.6 31.5) (size 0.6) (drill 0.3) (layers "F.Cu" "B.Cu") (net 4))
 (via (at 58.075 36) (size 0.6) (drill 0.3) (layers "F.Cu" "B.Cu") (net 4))
 (via (at 37.835586 29.86614) (size 0.6) (drill 0.3) (layers "F.Cu" "B.Cu") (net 4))
 (via (at 24.09995 36.8) (size 0.6) (drill 0.3) (layers "F.Cu" "B.Cu") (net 4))
 (via (at 46.310586 29.29114) (size 0.6) (drill 0.3) (layers "F.Cu" "B.Cu") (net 4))
 (via (at 28.310586 29.4) (size 0.6) (drill 0.3) (layers "F.Cu" "B.Cu") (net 4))
 (via (at 24.89995 36) (size 0.6) (drill 0.3) (layers "F.Cu" "B.Cu") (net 4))
 (via (at 34.585586 33.95614) (size 0.6) (drill 0.3) (layers "F.Cu" "B.Cu") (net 4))
 (segment (start 53.900586 37.86614) (end 52.396726 39.37) (width 0.6) (layer "F.Cu") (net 14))
 (segment (start 31.479446 39.37) (end 29.460586 37.35114) (width 0.6) (layer "F.Cu") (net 14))
 (segment (start 52.396726 39.37) (end 31.479446 39.37) (width 0.6) (layer "F.Cu") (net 14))
 (segment (start 29.460586 37.35114) (end 29.460586 35.54114) (width 0.6) (layer "F.Cu") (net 14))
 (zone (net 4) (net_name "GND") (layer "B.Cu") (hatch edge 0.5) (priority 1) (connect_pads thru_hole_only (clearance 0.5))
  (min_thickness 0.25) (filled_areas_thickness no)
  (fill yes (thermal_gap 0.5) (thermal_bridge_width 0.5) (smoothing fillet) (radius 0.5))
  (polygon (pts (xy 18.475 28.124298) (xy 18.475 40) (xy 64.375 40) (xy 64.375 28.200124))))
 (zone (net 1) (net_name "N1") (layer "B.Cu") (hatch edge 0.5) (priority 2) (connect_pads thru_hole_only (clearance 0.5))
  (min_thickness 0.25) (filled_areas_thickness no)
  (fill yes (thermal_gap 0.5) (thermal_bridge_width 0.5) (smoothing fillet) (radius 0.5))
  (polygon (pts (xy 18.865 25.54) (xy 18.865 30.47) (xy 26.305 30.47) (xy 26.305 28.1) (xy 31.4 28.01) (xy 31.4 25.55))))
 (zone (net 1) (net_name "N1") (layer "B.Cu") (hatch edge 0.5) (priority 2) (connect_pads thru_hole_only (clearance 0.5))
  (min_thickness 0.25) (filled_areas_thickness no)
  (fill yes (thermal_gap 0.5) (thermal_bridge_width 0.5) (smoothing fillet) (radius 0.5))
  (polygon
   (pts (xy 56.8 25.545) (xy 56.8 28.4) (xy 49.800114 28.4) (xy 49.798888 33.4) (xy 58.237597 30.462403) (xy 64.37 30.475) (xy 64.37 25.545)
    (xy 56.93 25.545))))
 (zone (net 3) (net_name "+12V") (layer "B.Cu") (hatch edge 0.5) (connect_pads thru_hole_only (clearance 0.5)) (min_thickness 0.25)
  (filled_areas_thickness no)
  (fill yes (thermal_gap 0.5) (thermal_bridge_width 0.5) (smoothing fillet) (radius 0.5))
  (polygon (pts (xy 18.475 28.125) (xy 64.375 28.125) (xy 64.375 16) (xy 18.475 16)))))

